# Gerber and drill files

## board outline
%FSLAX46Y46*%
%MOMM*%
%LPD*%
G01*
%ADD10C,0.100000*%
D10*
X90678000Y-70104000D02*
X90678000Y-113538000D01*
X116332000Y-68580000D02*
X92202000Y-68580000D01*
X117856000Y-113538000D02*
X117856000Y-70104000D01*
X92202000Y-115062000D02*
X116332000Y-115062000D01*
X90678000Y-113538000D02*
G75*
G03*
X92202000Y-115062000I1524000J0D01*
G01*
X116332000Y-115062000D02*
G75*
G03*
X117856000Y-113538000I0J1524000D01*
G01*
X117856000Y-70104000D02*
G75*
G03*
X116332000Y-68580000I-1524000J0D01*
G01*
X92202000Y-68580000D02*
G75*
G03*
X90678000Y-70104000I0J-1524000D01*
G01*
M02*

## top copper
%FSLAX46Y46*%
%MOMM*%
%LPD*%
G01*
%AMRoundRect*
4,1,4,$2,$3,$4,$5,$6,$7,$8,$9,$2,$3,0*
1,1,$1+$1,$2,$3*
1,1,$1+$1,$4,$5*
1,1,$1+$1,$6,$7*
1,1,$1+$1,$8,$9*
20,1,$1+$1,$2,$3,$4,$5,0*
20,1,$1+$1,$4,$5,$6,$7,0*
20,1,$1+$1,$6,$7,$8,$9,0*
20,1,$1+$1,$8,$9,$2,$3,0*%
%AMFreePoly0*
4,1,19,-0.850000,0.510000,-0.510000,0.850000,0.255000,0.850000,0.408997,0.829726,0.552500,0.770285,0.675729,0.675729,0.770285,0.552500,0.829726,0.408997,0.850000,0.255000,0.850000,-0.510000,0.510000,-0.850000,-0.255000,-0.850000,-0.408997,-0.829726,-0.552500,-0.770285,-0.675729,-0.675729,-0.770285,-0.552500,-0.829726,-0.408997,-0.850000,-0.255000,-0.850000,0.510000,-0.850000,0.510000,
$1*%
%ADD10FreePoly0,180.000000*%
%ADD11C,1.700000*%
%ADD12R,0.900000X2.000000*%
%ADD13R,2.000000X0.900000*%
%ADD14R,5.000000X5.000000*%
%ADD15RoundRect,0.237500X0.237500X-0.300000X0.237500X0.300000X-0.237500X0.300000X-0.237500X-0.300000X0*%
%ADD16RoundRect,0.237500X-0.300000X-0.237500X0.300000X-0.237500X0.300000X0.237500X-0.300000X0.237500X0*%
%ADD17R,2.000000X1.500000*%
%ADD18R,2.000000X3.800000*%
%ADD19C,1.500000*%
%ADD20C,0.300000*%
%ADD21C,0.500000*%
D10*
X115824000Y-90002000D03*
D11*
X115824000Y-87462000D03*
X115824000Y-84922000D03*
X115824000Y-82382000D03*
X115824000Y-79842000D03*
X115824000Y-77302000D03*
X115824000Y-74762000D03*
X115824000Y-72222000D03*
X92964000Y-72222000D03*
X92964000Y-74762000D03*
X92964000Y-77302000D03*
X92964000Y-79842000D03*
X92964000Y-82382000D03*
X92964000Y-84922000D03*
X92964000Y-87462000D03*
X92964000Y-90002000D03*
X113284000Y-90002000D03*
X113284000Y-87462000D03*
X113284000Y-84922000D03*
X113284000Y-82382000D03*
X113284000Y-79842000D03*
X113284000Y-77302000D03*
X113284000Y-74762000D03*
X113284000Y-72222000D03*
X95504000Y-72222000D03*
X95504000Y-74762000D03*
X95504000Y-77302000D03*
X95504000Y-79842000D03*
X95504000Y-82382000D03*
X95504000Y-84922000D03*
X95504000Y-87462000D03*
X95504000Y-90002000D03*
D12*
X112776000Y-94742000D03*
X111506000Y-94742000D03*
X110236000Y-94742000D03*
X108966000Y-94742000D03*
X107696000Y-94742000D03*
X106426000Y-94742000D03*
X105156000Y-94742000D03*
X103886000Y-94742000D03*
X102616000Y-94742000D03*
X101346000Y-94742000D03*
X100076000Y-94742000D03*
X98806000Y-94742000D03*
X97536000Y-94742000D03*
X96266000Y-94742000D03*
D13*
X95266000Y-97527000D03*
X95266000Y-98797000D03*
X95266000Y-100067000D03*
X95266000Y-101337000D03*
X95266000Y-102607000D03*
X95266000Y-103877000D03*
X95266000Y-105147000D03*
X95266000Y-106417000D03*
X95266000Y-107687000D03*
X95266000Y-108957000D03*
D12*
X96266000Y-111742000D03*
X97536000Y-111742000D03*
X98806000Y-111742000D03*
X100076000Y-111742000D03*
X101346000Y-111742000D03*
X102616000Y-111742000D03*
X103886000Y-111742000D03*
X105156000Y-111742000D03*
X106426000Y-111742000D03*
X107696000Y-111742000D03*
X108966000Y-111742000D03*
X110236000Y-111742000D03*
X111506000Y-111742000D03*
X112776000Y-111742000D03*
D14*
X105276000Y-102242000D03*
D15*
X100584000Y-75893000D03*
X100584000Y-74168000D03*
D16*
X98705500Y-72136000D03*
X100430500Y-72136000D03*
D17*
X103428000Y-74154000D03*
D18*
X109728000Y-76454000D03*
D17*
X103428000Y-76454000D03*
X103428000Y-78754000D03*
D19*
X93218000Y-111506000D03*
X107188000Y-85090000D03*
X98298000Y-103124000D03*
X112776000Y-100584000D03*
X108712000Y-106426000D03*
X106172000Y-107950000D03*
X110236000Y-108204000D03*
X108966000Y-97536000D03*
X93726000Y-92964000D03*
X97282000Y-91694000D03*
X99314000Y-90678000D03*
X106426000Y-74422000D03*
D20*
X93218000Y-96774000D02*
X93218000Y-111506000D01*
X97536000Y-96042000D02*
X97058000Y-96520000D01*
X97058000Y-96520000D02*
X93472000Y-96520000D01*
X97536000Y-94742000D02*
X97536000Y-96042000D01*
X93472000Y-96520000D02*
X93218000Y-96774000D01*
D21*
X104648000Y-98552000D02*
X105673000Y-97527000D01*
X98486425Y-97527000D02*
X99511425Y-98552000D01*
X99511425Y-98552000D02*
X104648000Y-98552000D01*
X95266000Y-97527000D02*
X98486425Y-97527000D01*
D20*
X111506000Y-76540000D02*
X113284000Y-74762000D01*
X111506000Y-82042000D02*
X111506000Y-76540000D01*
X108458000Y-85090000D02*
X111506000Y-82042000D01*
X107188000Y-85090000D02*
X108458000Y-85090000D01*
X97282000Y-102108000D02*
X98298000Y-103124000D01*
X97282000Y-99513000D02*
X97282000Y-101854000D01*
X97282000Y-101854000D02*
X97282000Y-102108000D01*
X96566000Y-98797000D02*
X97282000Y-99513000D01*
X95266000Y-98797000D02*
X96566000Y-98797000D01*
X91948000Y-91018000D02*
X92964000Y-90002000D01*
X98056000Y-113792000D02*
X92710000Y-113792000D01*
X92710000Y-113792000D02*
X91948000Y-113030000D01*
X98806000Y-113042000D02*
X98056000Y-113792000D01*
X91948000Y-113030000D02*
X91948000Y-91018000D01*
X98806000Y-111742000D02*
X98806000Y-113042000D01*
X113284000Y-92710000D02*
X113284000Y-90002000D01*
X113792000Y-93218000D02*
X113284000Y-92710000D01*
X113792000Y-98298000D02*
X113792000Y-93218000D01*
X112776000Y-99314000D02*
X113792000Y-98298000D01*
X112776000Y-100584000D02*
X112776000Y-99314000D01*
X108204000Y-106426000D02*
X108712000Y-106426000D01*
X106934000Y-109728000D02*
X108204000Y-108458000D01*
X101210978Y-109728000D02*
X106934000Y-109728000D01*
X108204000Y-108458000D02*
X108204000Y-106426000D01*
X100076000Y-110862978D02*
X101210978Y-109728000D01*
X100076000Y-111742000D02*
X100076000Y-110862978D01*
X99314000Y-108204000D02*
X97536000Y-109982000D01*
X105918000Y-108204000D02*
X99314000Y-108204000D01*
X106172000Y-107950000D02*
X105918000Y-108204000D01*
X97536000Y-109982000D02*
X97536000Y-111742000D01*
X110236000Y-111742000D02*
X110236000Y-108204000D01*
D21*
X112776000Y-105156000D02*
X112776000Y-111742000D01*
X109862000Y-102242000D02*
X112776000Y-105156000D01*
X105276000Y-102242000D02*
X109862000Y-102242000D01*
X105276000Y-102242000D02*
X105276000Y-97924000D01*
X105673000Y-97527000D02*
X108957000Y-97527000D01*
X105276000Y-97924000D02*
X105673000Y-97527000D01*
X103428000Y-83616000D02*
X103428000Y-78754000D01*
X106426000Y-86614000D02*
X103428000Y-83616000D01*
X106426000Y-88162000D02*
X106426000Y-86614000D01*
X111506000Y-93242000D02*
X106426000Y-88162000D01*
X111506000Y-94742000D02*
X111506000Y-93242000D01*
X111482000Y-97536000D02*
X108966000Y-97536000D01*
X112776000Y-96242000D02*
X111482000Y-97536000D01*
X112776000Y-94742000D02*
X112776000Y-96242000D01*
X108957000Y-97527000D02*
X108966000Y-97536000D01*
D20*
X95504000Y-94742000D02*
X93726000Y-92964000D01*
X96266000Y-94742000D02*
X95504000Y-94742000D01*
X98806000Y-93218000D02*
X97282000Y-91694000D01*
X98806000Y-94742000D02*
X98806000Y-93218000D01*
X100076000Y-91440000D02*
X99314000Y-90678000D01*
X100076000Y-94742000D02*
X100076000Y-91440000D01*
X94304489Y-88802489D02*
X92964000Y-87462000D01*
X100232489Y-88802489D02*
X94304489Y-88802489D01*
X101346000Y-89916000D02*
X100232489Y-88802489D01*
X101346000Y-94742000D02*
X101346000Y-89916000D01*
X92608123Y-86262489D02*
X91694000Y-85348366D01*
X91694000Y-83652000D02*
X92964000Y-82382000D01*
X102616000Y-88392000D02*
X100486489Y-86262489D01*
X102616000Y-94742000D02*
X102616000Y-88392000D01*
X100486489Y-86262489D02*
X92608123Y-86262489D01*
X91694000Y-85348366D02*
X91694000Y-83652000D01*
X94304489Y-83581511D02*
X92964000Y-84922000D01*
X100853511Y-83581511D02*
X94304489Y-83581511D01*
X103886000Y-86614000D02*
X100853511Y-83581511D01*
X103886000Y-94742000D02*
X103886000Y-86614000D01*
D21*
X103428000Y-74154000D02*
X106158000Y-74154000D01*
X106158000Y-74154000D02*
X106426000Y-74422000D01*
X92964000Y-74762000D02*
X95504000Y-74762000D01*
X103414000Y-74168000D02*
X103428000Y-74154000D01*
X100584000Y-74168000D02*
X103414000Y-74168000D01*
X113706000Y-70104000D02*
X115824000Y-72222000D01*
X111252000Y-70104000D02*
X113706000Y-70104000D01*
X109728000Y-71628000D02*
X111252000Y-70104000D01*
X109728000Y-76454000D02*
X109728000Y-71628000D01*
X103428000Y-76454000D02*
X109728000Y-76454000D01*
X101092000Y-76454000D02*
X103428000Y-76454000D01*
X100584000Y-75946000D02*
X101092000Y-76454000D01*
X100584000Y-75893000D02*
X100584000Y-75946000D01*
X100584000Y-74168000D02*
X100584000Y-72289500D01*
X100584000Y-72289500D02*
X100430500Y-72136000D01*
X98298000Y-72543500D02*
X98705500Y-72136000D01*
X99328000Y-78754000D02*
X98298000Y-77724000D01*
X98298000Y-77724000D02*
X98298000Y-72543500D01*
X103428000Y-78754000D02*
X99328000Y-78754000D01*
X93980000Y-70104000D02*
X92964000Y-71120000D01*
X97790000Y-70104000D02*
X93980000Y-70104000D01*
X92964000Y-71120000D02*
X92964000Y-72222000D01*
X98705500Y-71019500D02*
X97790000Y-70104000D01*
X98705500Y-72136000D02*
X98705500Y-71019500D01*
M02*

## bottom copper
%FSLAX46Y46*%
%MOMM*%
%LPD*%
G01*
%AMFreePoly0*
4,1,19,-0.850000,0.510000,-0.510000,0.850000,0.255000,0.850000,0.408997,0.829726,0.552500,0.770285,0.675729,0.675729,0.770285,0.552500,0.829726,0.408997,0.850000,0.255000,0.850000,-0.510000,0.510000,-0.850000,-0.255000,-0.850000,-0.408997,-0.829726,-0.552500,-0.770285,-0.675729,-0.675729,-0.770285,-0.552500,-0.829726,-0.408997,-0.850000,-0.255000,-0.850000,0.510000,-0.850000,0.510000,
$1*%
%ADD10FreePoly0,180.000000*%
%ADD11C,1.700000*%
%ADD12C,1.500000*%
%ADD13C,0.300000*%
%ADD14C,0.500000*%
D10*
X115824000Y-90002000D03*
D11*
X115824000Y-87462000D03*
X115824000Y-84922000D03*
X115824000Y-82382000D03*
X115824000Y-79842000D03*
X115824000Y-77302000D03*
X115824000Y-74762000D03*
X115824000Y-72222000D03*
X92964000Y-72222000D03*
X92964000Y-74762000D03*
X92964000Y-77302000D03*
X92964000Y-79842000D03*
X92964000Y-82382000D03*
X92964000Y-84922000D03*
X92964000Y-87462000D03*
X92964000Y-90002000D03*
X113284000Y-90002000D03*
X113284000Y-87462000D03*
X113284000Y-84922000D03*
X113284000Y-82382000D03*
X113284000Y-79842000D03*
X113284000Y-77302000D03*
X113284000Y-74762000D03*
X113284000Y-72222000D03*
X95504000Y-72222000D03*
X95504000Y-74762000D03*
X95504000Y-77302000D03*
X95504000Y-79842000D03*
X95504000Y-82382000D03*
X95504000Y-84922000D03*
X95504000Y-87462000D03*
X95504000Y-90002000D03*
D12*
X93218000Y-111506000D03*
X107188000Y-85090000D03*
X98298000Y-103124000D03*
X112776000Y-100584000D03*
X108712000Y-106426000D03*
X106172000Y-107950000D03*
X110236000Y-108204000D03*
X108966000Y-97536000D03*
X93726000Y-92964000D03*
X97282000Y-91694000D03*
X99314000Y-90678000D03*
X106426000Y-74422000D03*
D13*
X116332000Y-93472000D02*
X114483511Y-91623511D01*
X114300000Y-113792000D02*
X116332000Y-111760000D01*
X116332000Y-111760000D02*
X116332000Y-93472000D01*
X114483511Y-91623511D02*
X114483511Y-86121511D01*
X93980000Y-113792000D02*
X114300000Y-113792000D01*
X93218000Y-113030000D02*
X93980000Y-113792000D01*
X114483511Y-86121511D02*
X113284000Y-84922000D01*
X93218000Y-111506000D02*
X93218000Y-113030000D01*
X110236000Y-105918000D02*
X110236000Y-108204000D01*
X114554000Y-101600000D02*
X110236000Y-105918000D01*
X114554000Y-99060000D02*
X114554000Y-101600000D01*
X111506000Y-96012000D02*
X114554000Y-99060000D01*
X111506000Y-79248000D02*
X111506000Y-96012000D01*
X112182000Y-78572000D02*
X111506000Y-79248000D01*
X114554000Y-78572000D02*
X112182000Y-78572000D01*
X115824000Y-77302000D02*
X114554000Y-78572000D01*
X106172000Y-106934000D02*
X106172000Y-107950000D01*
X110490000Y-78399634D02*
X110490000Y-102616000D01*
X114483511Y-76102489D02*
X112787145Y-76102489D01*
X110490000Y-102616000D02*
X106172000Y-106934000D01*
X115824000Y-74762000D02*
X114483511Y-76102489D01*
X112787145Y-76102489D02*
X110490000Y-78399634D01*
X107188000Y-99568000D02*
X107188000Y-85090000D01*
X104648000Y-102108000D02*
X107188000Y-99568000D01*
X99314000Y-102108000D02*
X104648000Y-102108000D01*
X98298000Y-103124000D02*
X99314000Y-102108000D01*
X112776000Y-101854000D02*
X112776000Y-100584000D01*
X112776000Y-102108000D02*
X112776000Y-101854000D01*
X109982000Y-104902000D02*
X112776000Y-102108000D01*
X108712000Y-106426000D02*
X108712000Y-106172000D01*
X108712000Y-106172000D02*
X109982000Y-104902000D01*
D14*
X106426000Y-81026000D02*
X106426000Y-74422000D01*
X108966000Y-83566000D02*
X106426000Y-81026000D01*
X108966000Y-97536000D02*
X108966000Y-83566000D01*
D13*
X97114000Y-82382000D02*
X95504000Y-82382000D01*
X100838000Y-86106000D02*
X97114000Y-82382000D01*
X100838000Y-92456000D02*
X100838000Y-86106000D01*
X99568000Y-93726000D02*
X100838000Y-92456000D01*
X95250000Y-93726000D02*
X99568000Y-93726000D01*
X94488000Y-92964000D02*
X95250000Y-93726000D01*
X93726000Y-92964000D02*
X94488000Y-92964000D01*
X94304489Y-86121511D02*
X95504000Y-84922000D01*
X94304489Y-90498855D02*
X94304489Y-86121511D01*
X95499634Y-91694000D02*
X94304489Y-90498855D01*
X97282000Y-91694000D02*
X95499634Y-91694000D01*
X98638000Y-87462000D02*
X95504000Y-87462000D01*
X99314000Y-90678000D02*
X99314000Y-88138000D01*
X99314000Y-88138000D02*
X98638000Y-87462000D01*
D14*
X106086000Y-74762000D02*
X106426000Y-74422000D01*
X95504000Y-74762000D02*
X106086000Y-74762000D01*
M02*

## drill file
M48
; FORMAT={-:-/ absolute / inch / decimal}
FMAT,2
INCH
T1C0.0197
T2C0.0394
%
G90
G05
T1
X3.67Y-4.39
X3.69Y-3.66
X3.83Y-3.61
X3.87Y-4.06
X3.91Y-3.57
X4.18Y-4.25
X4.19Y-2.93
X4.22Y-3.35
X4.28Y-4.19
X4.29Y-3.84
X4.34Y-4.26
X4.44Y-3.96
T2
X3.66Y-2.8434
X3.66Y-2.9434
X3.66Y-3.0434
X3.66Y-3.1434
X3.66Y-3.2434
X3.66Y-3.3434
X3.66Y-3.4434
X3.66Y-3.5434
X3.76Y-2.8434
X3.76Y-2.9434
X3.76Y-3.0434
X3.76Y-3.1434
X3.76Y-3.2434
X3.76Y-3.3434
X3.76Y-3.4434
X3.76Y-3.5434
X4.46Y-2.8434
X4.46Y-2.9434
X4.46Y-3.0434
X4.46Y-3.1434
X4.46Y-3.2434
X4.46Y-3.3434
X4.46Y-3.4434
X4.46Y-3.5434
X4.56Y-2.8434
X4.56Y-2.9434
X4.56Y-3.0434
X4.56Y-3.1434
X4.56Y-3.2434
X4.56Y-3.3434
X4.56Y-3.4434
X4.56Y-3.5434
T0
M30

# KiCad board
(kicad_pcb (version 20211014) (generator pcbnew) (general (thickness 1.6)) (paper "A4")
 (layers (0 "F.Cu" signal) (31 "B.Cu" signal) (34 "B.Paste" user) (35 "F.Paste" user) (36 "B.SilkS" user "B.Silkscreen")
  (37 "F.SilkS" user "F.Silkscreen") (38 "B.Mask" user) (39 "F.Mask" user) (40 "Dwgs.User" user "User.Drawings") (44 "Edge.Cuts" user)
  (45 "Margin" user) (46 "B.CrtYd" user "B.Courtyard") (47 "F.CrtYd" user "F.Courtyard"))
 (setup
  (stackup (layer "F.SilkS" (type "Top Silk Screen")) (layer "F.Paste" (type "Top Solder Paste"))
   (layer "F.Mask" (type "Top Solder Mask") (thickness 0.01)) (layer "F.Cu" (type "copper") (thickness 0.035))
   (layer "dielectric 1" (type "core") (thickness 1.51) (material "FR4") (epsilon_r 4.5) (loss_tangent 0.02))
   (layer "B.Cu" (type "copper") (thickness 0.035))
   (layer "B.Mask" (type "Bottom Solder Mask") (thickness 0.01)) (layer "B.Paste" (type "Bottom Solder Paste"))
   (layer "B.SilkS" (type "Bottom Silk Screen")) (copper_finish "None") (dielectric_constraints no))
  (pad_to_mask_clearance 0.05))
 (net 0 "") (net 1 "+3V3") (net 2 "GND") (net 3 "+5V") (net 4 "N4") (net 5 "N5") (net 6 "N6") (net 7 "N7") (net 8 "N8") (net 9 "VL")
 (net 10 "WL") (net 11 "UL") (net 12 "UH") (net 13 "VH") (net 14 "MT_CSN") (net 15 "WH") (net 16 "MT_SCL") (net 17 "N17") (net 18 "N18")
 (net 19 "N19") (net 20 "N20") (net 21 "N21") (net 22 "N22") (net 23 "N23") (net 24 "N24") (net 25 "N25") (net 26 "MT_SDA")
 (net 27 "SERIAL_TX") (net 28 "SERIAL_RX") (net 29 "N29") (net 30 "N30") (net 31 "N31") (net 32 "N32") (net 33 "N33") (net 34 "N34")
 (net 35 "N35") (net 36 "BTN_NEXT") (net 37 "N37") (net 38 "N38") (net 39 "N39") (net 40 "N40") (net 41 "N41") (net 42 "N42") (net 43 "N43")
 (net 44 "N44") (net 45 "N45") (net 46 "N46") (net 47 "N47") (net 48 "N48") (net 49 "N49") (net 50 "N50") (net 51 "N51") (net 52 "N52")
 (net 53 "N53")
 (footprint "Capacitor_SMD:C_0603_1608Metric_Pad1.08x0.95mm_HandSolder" (layer "F.Cu") (at 100.584 75.0305 90)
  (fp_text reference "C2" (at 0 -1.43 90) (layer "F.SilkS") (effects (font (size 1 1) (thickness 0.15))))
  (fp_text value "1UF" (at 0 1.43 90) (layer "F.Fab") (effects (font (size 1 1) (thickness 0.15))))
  (pad "1" smd roundrect (at -0.8625 0 90) (size 1.075 0.95) (layers "F.Cu" "F.Paste" "F.Mask") (roundrect_rratio 0.25) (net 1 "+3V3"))
  (pad "2" smd roundrect (at 0.8625 0 90) (size 1.075 0.95) (layers "F.Cu" "F.Paste" "F.Mask") (roundrect_rratio 0.25) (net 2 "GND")))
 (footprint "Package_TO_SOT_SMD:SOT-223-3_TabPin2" (layer "F.Cu") (at 106.578 76.454)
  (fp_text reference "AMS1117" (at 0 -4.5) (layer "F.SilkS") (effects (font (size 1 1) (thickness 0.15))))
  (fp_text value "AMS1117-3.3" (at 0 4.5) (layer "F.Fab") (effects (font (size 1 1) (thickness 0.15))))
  (pad "1" smd rect (at -3.15 -2.3) (size 2 1.5) (layers "F.Cu" "F.Paste" "F.Mask") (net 2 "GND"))
  (pad "2" smd rect (at -3.15 0) (size 2 1.5) (layers "F.Cu" "F.Paste" "F.Mask") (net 1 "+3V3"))
  (pad "2" smd rect (at 3.15 0) (size 2 3.8) (layers "F.Cu" "F.Paste" "F.Mask") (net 1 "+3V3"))
  (pad "3" smd rect (at -3.15 2.3) (size 2 1.5) (layers "F.Cu" "F.Paste" "F.Mask") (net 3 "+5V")))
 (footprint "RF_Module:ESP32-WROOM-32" (layer "F.Cu") (at 104.521 103.242 -90)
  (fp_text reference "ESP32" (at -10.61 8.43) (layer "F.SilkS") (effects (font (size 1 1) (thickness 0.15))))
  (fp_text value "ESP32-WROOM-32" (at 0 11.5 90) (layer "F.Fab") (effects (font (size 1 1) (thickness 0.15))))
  (pad "1" smd rect (at -8.5 -8.255 270) (size 2 0.9) (layers "F.Cu" "F.Paste" "F.Mask") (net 2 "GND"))
  (pad "2" smd rect (at -8.5 -6.985 270) (size 2 0.9) (layers "F.Cu" "F.Paste" "F.Mask") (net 3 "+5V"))
  (pad "3" smd rect (at -8.5 -5.715 270) (size 2 0.9) (layers "F.Cu" "F.Paste" "F.Mask") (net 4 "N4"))
  (pad "4" smd rect (at -8.5 -4.445 270) (size 2 0.9) (layers "F.Cu" "F.Paste" "F.Mask") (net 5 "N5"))
  (pad "5" smd rect (at -8.5 -3.175 270) (size 2 0.9) (layers "F.Cu" "F.Paste" "F.Mask") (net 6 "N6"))
  (pad "6" smd rect (at -8.5 -1.905 270) (size 2 0.9) (layers "F.Cu" "F.Paste" "F.Mask") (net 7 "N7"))
  (pad "7" smd rect (at -8.5 -0.635 270) (size 2 0.9) (layers "F.Cu" "F.Paste" "F.Mask") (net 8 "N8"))
  (pad "8" smd rect (at -8.5 0.635 270) (size 2 0.9) (layers "F.Cu" "F.Paste" "F.Mask") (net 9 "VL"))
  (pad "9" smd rect (at -8.5 1.905 270) (size 2 0.9) (layers "F.Cu" "F.Paste" "F.Mask") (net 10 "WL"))
  (pad "10" smd rect (at -8.5 3.175 270) (size 2 0.9) (layers "F.Cu" "F.Paste" "F.Mask") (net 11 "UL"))
  (pad "11" smd rect (at -8.5 4.445 270) (size 2 0.9) (layers "F.Cu" "F.Paste" "F.Mask") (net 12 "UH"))
  (pad "12" smd rect (at -8.5 5.715 270) (size 2 0.9) (layers "F.Cu" "F.Paste" "F.Mask") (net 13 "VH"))
  (pad "13" smd rect (at -8.5 6.985 270) (size 2 0.9) (layers "F.Cu" "F.Paste" "F.Mask") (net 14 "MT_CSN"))
  (pad "14" smd rect (at -8.5 8.255 270) (size 2 0.9) (layers "F.Cu" "F.Paste" "F.Mask") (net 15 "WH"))
  (pad "15" smd rect (at -5.715 9.255) (size 2 0.9) (layers "F.Cu" "F.Paste" "F.Mask") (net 2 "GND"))
  (pad "16" smd rect (at -4.445 9.255) (size 2 0.9) (layers "F.Cu" "F.Paste" "F.Mask") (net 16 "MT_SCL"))
  (pad "17" smd rect (at -3.175 9.255) (size 2 0.9) (layers "F.Cu" "F.Paste" "F.Mask") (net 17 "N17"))
  (pad "18" smd rect (at -1.905 9.255) (size 2 0.9) (layers "F.Cu" "F.Paste" "F.Mask") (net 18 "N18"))
  (pad "19" smd rect (at -0.635 9.255) (size 2 0.9) (layers "F.Cu" "F.Paste" "F.Mask") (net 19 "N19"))
  (pad "20" smd rect (at 0.635 9.255) (size 2 0.9) (layers "F.Cu" "F.Paste" "F.Mask") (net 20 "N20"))
  (pad "21" smd rect (at 1.905 9.255) (size 2 0.9) (layers "F.Cu" "F.Paste" "F.Mask") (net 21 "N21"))
  (pad "22" smd rect (at 3.175 9.255) (size 2 0.9) (layers "F.Cu" "F.Paste" "F.Mask") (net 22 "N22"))
  (pad "23" smd rect (at 4.445 9.255) (size 2 0.9) (layers "F.Cu" "F.Paste" "F.Mask") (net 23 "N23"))
  (pad "24" smd rect (at 5.715 9.255) (size 2 0.9) (layers "F.Cu" "F.Paste" "F.Mask") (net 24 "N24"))
  (pad "25" smd rect (at 8.5 8.255 270) (size 2 0.9) (layers "F.Cu" "F.Paste" "F.Mask") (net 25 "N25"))
  (pad "26" smd rect (at 8.5 6.985 270) (size 2 0.9) (layers "F.Cu" "F.Paste" "F.Mask") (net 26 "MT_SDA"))
  (pad "27" smd rect (at 8.5 5.715 270) (size 2 0.9) (layers "F.Cu" "F.Paste" "F.Mask") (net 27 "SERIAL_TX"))
  (pad "28" smd rect (at 8.5 4.445 270) (size 2 0.9) (layers "F.Cu" "F.Paste" "F.Mask") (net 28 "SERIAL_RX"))
  (pad "29" smd rect (at 8.5 3.175 270) (size 2 0.9) (layers "F.Cu" "F.Paste" "F.Mask") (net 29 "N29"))
  (pad "30" smd rect (at 8.5 1.905 270) (size 2 0.9) (layers "F.Cu" "F.Paste" "F.Mask") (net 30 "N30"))
  (pad "31" smd rect (at 8.5 0.635 270) (size 2 0.9) (layers "F.Cu" "F.Paste" "F.Mask") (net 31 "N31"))
  (pad "32" smd rect (at 8.5 -0.635 270) (size 2 0.9) (layers "F.Cu" "F.Paste" "F.Mask") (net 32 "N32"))
  (pad "33" smd rect (at 8.5 -1.905 270) (size 2 0.9) (layers "F.Cu" "F.Paste" "F.Mask") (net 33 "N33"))
  (pad "34" smd rect (at 8.5 -3.175 270) (size 2 0.9) (layers "F.Cu" "F.Paste" "F.Mask") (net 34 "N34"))
  (pad "35" smd rect (at 8.5 -4.445 270) (size 2 0.9) (layers "F.Cu" "F.Paste" "F.Mask") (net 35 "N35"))
  (pad "36" smd rect (at 8.5 -5.715 270) (size 2 0.9) (layers "F.Cu" "F.Paste" "F.Mask") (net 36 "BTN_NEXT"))
  (pad "37" smd rect (at 8.5 -6.985 270) (size 2 0.9) (layers "F.Cu" "F.Paste" "F.Mask") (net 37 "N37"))
  (pad "38" smd rect (at 8.5 -8.255 270) (size 2 0.9) (layers "F.Cu" "F.Paste" "F.Mask") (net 2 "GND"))
  (pad "39" smd rect (at -1 -0.755 270) (size 5 5) (layers "F.Cu" "F.Paste" "F.Mask") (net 2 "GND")))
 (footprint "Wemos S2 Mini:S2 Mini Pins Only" (layer "F.Cu") (at 104.394 79.502 180)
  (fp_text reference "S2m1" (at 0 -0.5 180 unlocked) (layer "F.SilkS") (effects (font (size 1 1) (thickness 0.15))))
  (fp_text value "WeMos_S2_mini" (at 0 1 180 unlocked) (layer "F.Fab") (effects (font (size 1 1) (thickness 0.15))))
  (pad "1" thru_hole roundrect (at -11.43 -10.5 180) (size 1.7 1.7) (drill 1) (layers *.Cu *.Mask) (roundrect_rratio 0.35)
   (chamfer_ratio 0.2) (chamfer top_left bottom_right) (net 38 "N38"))
  (pad "2" thru_hole circle (at -11.43 -7.96 180) (size 1.7 1.7) (drill 1) (layers *.Cu *.Mask) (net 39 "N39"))
  (pad "3" thru_hole circle (at -11.43 -5.42 180) (size 1.7 1.7) (drill 1) (layers *.Cu *.Mask) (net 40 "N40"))
  (pad "4" thru_hole circle (at -11.43 -2.88 180) (size 1.7 1.7) (drill 1) (layers *.Cu *.Mask) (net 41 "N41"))
  (pad "5" thru_hole circle (at -11.43 -0.34 180) (size 1.7 1.7) (drill 1) (layers *.Cu *.Mask) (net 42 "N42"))
  (pad "6" thru_hole circle (at -11.43 2.2 180) (size 1.7 1.7) (drill 1) (layers *.Cu *.Mask) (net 36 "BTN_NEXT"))
  (pad "7" thru_hole circle (at -11.43 4.74 180) (size 1.7 1.7) (drill 1) (layers *.Cu *.Mask) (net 26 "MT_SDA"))
  (pad "8" thru_hole circle (at -11.43 7.28 180) (size 1.7 1.7) (drill 1) (layers *.Cu *.Mask) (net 1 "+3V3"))
  (pad "9" thru_hole circle (at 11.43 7.28 180) (size 1.7 1.7) (drill 1) (layers *.Cu *.Mask) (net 3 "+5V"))
  (pad "10" thru_hole circle (at 11.43 4.74 180) (size 1.7 1.7) (drill 1) (layers *.Cu *.Mask) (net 2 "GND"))
  (pad "11" thru_hole circle (at 11.43 2.2 180) (size 1.7 1.7) (drill 1) (layers *.Cu *.Mask) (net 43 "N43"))
  (pad "12" thru_hole circle (at 11.43 -0.34 180) (size 1.7 1.7) (drill 1) (layers *.Cu *.Mask) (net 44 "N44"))
  (pad "13" thru_hole circle (at 11.43 -2.88 180) (size 1.7 1.7) (drill 1) (layers *.Cu *.Mask) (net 10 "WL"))
  (pad "14" thru_hole circle (at 11.43 -5.42 180) (size 1.7 1.7) (drill 1) (layers *.Cu *.Mask) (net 9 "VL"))
  (pad "15" thru_hole circle (at 11.43 -7.96 180) (size 1.7 1.7) (drill 1) (layers *.Cu *.Mask) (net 11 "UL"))
  (pad "16" thru_hole circle (at 11.43 -10.5 180) (size 1.7 1.7) (drill 1) (layers *.Cu *.Mask) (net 27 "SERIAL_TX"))
  (pad "17" thru_hole circle (at -8.89 -10.5 180) (size 1.7 1.7) (drill 1) (layers *.Cu *.Mask) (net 28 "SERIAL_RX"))
  (pad "18" thru_hole circle (at -8.89 -7.96 180) (size 1.7 1.7) (drill 1) (layers *.Cu *.Mask) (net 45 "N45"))
  (pad "19" thru_hole circle (at -8.89 -5.42 180) (size 1.7 1.7) (drill 1) (layers *.Cu *.Mask) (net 14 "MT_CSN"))
  (pad "20" thru_hole circle (at -8.89 -2.88 180) (size 1.7 1.7) (drill 1) (layers *.Cu *.Mask) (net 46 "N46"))
  (pad "21" thru_hole circle (at -8.89 -0.34 180) (size 1.7 1.7) (drill 1) (layers *.Cu *.Mask) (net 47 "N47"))
  (pad "22" thru_hole circle (at -8.89 2.2 180) (size 1.7 1.7) (drill 1) (layers *.Cu *.Mask) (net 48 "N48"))
  (pad "23" thru_hole circle (at -8.89 4.74 180) (size 1.7 1.7) (drill 1) (layers *.Cu *.Mask) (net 16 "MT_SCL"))
  (pad "24" thru_hole circle (at -8.89 7.28 180) (size 1.7 1.7) (drill 1) (layers *.Cu *.Mask) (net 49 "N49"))
  (pad "25" thru_hole circle (at 8.89 7.28 180) (size 1.7 1.7) (drill 1) (layers *.Cu *.Mask) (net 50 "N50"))
  (pad "26" thru_hole circle (at 8.89 4.74 180) (size 1.7 1.7) (drill 1) (layers *.Cu *.Mask) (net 2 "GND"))
  (pad "27" thru_hole circle (at 8.89 2.2 180) (size 1.7 1.7) (drill 1) (layers *.Cu *.Mask) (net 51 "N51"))
  (pad "28" thru_hole circle (at 8.89 -0.34 180) (size 1.7 1.7) (drill 1) (layers *.Cu *.Mask) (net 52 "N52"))
  (pad "29" thru_hole circle (at 8.89 -2.88 180) (size 1.7 1.7) (drill 1) (layers *.Cu *.Mask) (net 15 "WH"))
  (pad "30" thru_hole circle (at 8.89 -5.42 180) (size 1.7 1.7) (drill 1) (layers *.Cu *.Mask) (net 13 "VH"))
  (pad "31" thru_hole circle (at 8.89 -7.96 180) (size 1.7 1.7) (drill 1) (layers *.Cu *.Mask) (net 12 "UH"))
  (pad "32" thru_hole circle (at 8.89 -10.5 180) (size 1.7 1.7) (drill 1) (layers *.Cu *.Mask) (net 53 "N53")))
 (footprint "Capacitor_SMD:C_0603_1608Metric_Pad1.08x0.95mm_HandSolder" (layer "F.Cu") (at 99.568 72.136)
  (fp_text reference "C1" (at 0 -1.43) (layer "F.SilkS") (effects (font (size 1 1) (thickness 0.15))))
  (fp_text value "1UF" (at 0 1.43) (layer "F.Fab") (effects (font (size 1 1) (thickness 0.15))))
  (pad "1" smd roundrect (at -0.8625 0) (size 1.075 0.95) (layers "F.Cu" "F.Paste" "F.Mask") (roundrect_rratio 0.25) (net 3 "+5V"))
  (pad "2" smd roundrect (at 0.8625 0) (size 1.075 0.95) (layers "F.Cu" "F.Paste" "F.Mask") (roundrect_rratio 0.25) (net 2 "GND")))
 (gr_arc (start 117.856 113.538) (mid 117.409631 114.615631) (end 116.332 115.062) (layer "Edge.Cuts") (width 0.1))
 (gr_arc (start 90.678 70.104) (mid 91.124369 69.026369) (end 92.202 68.58) (layer "Edge.Cuts") (width 0.1))
 (gr_line (start 90.678 70.104) (end 90.678 113.538) (layer "Edge.Cuts") (width 0.1))
 (gr_arc (start 116.332 68.58) (mid 117.409631 69.026369) (end 117.856 70.104) (layer "Edge.Cuts") (width 0.1))
 (gr_line (start 92.202 115.062) (end 116.332 115.062) (layer "Edge.Cuts") (width 0.1))
 (gr_line (start 117.856 113.538) (end 117.856 70.104) (layer "Edge.Cuts") (width 0.1))
 (gr_line (start 116.332 68.58) (end 92.202 68.58) (layer "Edge.Cuts") (width 0.1))
 (gr_arc (start 92.202 115.062) (mid 91.124369 114.615631) (end 90.678 113.538) (layer "Edge.Cuts") (width 0.1))
 (segment (start 106.158 74.154) (end 106.426 74.422) (width 0.5) (layer "F.Cu") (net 2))
 (segment (start 99.511425 98.552) (end 104.648 98.552) (width 0.5) (layer "F.Cu") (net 2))
 (segment (start 98.486425 97.527) (end 99.511425 98.552) (width 0.5) (layer "F.Cu") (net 2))
 (segment (start 103.414 74.168) (end 103.428 74.154) (width 0.5) (layer "F.Cu") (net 2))
 (segment (start 112.776 105.156) (end 112.776 111.742) (width 0.5) (layer "F.Cu") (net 2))
 (segment (start 105.276 97.924) (end 105.673 97.527) (width 0.5) (layer "F.Cu") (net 2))
 (segment (start 100.584 74.168) (end 100.584 72.2895) (width 0.5) (layer "F.Cu") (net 2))
 (segment (start 104.648 98.552) (end 105.673 97.527) (width 0.5) (layer "F.Cu") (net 2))
 (segment (start 105.673 97.527) (end 108.957 97.527) (width 0.5) (layer "F.Cu") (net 2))
 (segment (start 100.584 72.2895) (end 100.4305 72.136) (width 0.5) (layer "F.Cu") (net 2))
 (segment (start 103.428 74.154) (end 106.158 74.154) (width 0.5) (layer "F.Cu") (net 2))
 (segment (start 112.776 96.242) (end 111.482 97.536) (width 0.5) (layer "F.Cu") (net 2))
 (segment (start 109.862 102.242) (end 112.776 105.156) (width 0.5) (layer "F.Cu") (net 2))
 (segment (start 111.482 97.536) (end 108.966 97.536) (width 0.5) (layer "F.Cu") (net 2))
 (segment (start 92.964 74.762) (end 95.504 74.762) (width 0.5) (layer "F.Cu") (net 2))
 (segment (start 112.776 94.742) (end 112.776 96.242) (width 0.5) (layer "F.Cu") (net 2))
 (segment (start 108.957 97.527) (end 108.966 97.536) (width 0.5) (layer "F.Cu") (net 2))
 (segment (start 100.584 74.168) (end 103.414 74.168) (width 0.5) (layer "F.Cu") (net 2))
 (segment (start 95.266 97.527) (end 98.486425 97.527) (width 0.5) (layer "F.Cu") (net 2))
 (segment (start 105.276 102.242) (end 105.276 97.924) (width 0.5) (layer "F.Cu") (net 2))
 (segment (start 105.276 102.242) (end 109.862 102.242) (width 0.5) (layer "F.Cu") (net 2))
 (via (at 106.426 74.422) (size 1.5) (drill 0.5) (layers "F.Cu" "B.Cu") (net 2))
 (via (at 108.966 97.536) (size 1.5) (drill 0.5) (layers "F.Cu" "B.Cu") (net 2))
 (segment (start 106.086 74.762) (end 106.426 74.422) (width 0.5) (layer "B.Cu") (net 2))
 (segment (start 108.966 97.536) (end 108.966 83.566) (width 0.5) (layer "B.Cu") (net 2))
 (segment (start 95.504 74.762) (end 106.086 74.762) (width 0.5) (layer "B.Cu") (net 2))
 (segment (start 108.966 83.566) (end 106.426 81.026) (width 0.5) (layer "B.Cu") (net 2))
 (segment (start 106.426 81.026) (end 106.426 74.422) (width 0.5) (layer "B.Cu") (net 2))
 (segment (start 109.728 76.454) (end 109.728 71.628) (width 0.5) (layer "F.Cu") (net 1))
 (segment (start 111.252 70.104) (end 113.706 70.104) (width 0.5) (layer "F.Cu") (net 1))
 (segment (start 109.728 71.628) (end 111.252 70.104) (width 0.5) (layer "F.Cu") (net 1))
 (segment (start 101.092 76.454) (end 103.428 76.454) (width 0.5) (layer "F.Cu") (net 1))
 (segment (start 103.428 76.454) (end 109.728 76.454) (width 0.5) (layer "F.Cu") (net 1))
 (segment (start 100.584 75.893) (end 100.584 75.946) (width 0.5) (layer "F.Cu") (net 1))
 (segment (start 100.584 75.946) (end 101.092 76.454) (width 0.5) (layer "F.Cu") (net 1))
 (segment (start 113.706 70.104) (end 115.824 72.222) (width 0.5) (layer "F.Cu") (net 1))
 (segment (start 98.298 77.724) (end 98.298 72.5435) (width 0.5) (layer "F.Cu") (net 3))
 (segment (start 111.506 93.242) (end 106.426 88.162) (width 0.5) (layer "F.Cu") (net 3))
 (segment (start 93.98 70.104) (end 92.964 71.12) (width 0.5) (layer "F.Cu") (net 3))
 (segment (start 106.426 86.614) (end 103.428 83.616) (width 0.5) (layer "F.Cu") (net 3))
 (segment (start 92.964 71.12) (end 92.964 72.222) (width 0.5) (layer "F.Cu") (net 3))
 (segment (start 111.506 94.742) (end 111.506 93.242) (width 0.5) (layer "F.Cu") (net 3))
 (segment (start 98.298 72.5435) (end 98.7055 72.136) (width 0.5) (layer "F.Cu") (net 3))
 (segment (start 103.428 78.754) (end 99.328 78.754) (width 0.5) (layer "F.Cu") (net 3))
 (segment (start 103.428 83.616) (end 103.428 78.754) (width 0.5) (layer "F.Cu") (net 3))
 (segment (start 106.426 88.162) (end 106.426 86.614) (width 0.5) (layer "F.Cu") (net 3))
 (segment (start 98.7055 71.0195) (end 97.79 70.104) (width 0.5) (layer "F.Cu") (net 3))
 (segment (start 98.7055 72.136) (end 98.7055 71.0195) (width 0.5) (layer "F.Cu") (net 3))
 (segment (start 97.79 70.104) (end 93.98 70.104) (width 0.5) (layer "F.Cu") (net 3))
 (segment (start 99.328 78.754) (end 98.298 77.724) (width 0.5) (layer "F.Cu") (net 3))
 (segment (start 100.853511 83.581511) (end 94.304489 83.581511) (width 0.3) (layer "F.Cu") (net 9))
 (segment (start 94.304489 83.581511) (end 92.964 84.922) (width 0.3) (layer "F.Cu") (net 9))
 (segment (start 103.886 86.614) (end 100.853511 83.581511) (width 0.3) (layer "F.Cu") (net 9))
 (segment (start 103.886 94.742) (end 103.886 86.614) (width 0.3) (layer "F.Cu") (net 9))
 (segment (start 92.608123 86.262489) (end 91.694 85.348366) (width 0.3) (layer "F.Cu") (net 10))
 (segment (start 91.694 85.348366) (end 91.694 83.652) (width 0.3) (layer "F.Cu") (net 10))
 (segment (start 91.694 83.652) (end 92.964 82.382) (width 0.3) (layer "F.Cu") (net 10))
 (segment (start 102.616 94.742) (end 102.616 88.392) (width 0.3) (layer "F.Cu") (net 10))
 (segment (start 100.486489 86.262489) (end 92.608123 86.262489) (width 0.3) (layer "F.Cu") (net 10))
 (segment (start 102.616 88.392) (end 100.486489 86.262489) (width 0.3) (layer "F.Cu") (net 10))
 (segment (start 101.346 94.742) (end 101.346 89.916) (width 0.3) (layer "F.Cu") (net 11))
 (segment (start 100.232489 88.802489) (end 94.304489 88.802489) (width 0.3) (layer "F.Cu") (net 11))
 (segment (start 94.304489 88.802489) (end 92.964 87.462) (width 0.3) (layer "F.Cu") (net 11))
 (segment (start 101.346 89.916) (end 100.232489 88.802489) (width 0.3) (layer "F.Cu") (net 11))
 (segment (start 100.076 91.44) (end 99.314 90.678) (width 0.3) (layer "F.Cu") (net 12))
 (segment (start 100.076 94.742) (end 100.076 91.44) (width 0.3) (layer "F.Cu") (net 12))
 (via (at 99.314 90.678) (size 1.5) (drill 0.5) (layers "F.Cu" "B.Cu") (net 12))
 (segment (start 98.638 87.462) (end 95.504 87.462) (width 0.3) (layer "B.Cu") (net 12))
 (segment (start 99.314 88.138) (end 98.638 87.462) (width 0.3) (layer "B.Cu") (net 12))
 (segment (start 99.314 90.678) (end 99.314 88.138) (width 0.3) (layer "B.Cu") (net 12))
 (segment (start 98.806 94.742) (end 98.806 93.218) (width 0.3) (layer "F.Cu") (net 13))
 (segment (start 98.806 93.218) (end 97.282 91.694) (width 0.3) (layer "F.Cu") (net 13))
 (via (at 97.282 91.694) (size 1.5) (drill 0.5) (layers "F.Cu" "B.Cu") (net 13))
 (segment (start 94.304489 90.498855) (end 94.304489 86.121511) (width 0.3) (layer "B.Cu") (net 13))
 (segment (start 95.499634 91.694) (end 94.304489 90.498855) (width 0.3) (layer "B.Cu") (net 13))
 (segment (start 97.282 91.694) (end 95.499634 91.694) (width 0.3) (layer "B.Cu") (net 13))
 (segment (start 94.304489 86.121511) (end 95.504 84.922) (width 0.3) (layer "B.Cu") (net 13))
 (segment (start 97.058 96.52) (end 93.472 96.52) (width 0.3) (layer "F.Cu") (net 14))
 (segment (start 93.472 96.52) (end 93.218 96.774) (width 0.3) (layer "F.Cu") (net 14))
 (segment (start 97.536 96.042) (end 97.058 96.52) (width 0.3) (layer "F.Cu") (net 14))
 (segment (start 97.536 94.742) (end 97.536 96.042) (width 0.3) (layer "F.Cu") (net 14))
 (segment (start 93.218 96.774) (end 93.218 111.506) (width 0.3) (layer "F.Cu") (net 14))
 (via (at 93.218 111.506) (size 1.5) (drill 0.5) (layers "F.Cu" "B.Cu") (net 14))
 (segment (start 93.218 111.506) (end 93.218 113.03) (width 0.3) (layer "B.Cu") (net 14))
 (segment (start 114.3 113.792) (end 116.332 111.76) (width 0.3) (layer "B.Cu") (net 14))
 (segment (start 116.332 93.472) (end 114.483511 91.623511) (width 0.3) (layer "B.Cu") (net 14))
 (segment (start 93.98 113.792) (end 114.3 113.792) (width 0.3) (layer "B.Cu") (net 14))
 (segment (start 114.483511 86.121511) (end 113.284 84.922) (width 0.3) (layer "B.Cu") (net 14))
 (segment (start 93.218 113.03) (end 93.98 113.792) (width 0.3) (layer "B.Cu") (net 14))
 (segment (start 114.483511 91.623511) (end 114.483511 86.121511) (width 0.3) (layer "B.Cu") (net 14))
 (segment (start 116.332 111.76) (end 116.332 93.472) (width 0.3) (layer "B.Cu") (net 14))
 (segment (start 96.266 94.742) (end 95.504 94.742) (width 0.3) (layer "F.Cu") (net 15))
 (segment (start 95.504 94.742) (end 93.726 92.964) (width 0.3) (layer "F.Cu") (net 15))
 (via (at 93.726 92.964) (size 1.5) (drill 0.5) (layers "F.Cu" "B.Cu") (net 15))
 (segment (start 100.838 86.106) (end 97.114 82.382) (width 0.3) (layer "B.Cu") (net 15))
 (segment (start 94.488 92.964) (end 95.25 93.726) (width 0.3) (layer "B.Cu") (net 15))
 (segment (start 99.568 93.726) (end 100.838 92.456) (width 0.3) (layer "B.Cu") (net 15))
 (segment (start 100.838 92.456) (end 100.838 86.106) (width 0.3) (layer "B.Cu") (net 15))
 (segment (start 93.726 92.964) (end 94.488 92.964) (width 0.3) (layer "B.Cu") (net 15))
 (segment (start 95.25 93.726) (end 99.568 93.726) (width 0.3) (layer "B.Cu") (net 15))
 (segment (start 97.114 82.382) (end 95.504 82.382) (width 0.3) (layer "B.Cu") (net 15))
 (segment (start 97.282 102.108) (end 98.298 103.124) (width 0.3) (layer "F.Cu") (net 16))
 (segment (start 111.506 82.042) (end 111.506 76.54) (width 0.3) (layer "F.Cu") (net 16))
 (segment (start 107.188 85.09) (end 108.458 85.09) (width 0.3) (layer "F.Cu") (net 16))
 (segment (start 97.282 101.854) (end 97.282 102.108) (width 0.3) (layer "F.Cu") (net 16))
 (segment (start 111.506 76.54) (end 113.284 74.762) (width 0.3) (layer "F.Cu") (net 16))
 (segment (start 95.266 98.797) (end 96.566 98.797) (width 0.3) (layer "F.Cu") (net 16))
 (segment (start 97.282 99.513) (end 97.282 101.854) (width 0.3) (layer "F.Cu") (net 16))
 (segment (start 108.458 85.09) (end 111.506 82.042) (width 0.3) (layer "F.Cu") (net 16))
 (segment (start 96.566 98.797) (end 97.282 99.513) (width 0.3) (layer "F.Cu") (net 16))
 (via (at 98.298 103.124) (size 1.5) (drill 0.5) (layers "F.Cu" "B.Cu") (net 16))
 (via (at 107.188 85.09) (size 1.5) (drill 0.5) (layers "F.Cu" "B.Cu") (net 16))
 (segment (start 99.314 102.108) (end 104.648 102.108) (width 0.3) (layer "B.Cu") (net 16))
 (segment (start 107.188 99.568) (end 107.188 85.09) (width 0.3) (layer "B.Cu") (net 16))
 (segment (start 104.648 102.108) (end 107.188 99.568) (width 0.3) (layer "B.Cu") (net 16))
 (segment (start 98.298 103.124) (end 99.314 102.108) (width 0.3) (layer "B.Cu") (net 16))
 (segment (start 105.918 108.204) (end 99.314 108.204) (width 0.3) (layer "F.Cu") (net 26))
 (segment (start 97.536 109.982) (end 97.536 111.742) (width 0.3) (layer "F.Cu") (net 26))
 (segment (start 106.172 107.95) (end 105.918 108.204) (width 0.3) (layer "F.Cu") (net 26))
 (segment (start 99.314 108.204) (end 97.536 109.982) (width 0.3) (layer "F.Cu") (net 26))
 (via (at 106.172 107.95) (size 1.5) (drill 0.5) (layers "F.Cu" "B.Cu") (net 26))
 (segment (start 110.49 102.616) (end 106.172 106.934) (width 0.3) (layer "B.Cu") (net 26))
 (segment (start 115.824 74.762) (end 114.483511 76.102489) (width 0.3) (layer "B.Cu") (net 26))
 (segment (start 112.787145 76.102489) (end 110.49 78.399634) (width 0.3) (layer "B.Cu") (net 26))
 (segment (start 114.483511 76.102489) (end 112.787145 76.102489) (width 0.3) (layer "B.Cu") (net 26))
 (segment (start 110.49 78.399634) (end 110.49 102.616) (width 0.3) (layer "B.Cu") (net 26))
 (segment (start 106.172 106.934) (end 106.172 107.95) (width 0.3) (layer "B.Cu") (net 26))
 (segment (start 98.056 113.792) (end 92.71 113.792) (width 0.3) (layer "F.Cu") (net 27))
 (segment (start 92.71 113.792) (end 91.948 113.03) (width 0.3) (layer "F.Cu") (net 27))
 (segment (start 91.948 91.018) (end 92.964 90.002) (width 0.3) (layer "F.Cu") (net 27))
 (segment (start 98.806 113.042) (end 98.056 113.792) (width 0.3) (layer "F.Cu") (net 27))
 (segment (start 98.806 111.742) (end 98.806 113.042) (width 0.3) (layer "F.Cu") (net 27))
 (segment (start 91.948 113.03) (end 91.948 91.018) (width 0.3) (layer "F.Cu") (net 27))
 (segment (start 108.204 108.458) (end 108.204 106.426) (width 0.3) (layer "F.Cu") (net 28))
 (segment (start 112.776 100.584) (end 112.776 99.314) (width 0.3) (layer "F.Cu") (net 28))
 (segment (start 113.284 92.71) (end 113.284 90.002) (width 0.3) (layer "F.Cu") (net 28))
 (segment (start 113.792 98.298) (end 113.792 93.218) (width 0.3) (layer "F.Cu") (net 28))
 (segment (start 112.776 99.314) (end 113.792 98.298) (width 0.3) (layer "F.Cu") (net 28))
 (segment (start 108.204 106.426) (end 108.712 106.426) (width 0.3) (layer "F.Cu") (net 28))
 (segment (start 100.076 110.862978) (end 101.210978 109.728) (width 0.3) (layer "F.Cu") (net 28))
 (segment (start 100.076 111.742) (end 100.076 110.862978) (width 0.3) (layer "F.Cu") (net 28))
 (segment (start 106.934 109.728) (end 108.204 108.458) (width 0.3) (layer "F.Cu") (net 28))
 (segment (start 101.210978 109.728) (end 106.934 109.728) (width 0.3) (layer "F.Cu") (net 28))
 (segment (start 113.792 93.218) (end 113.284 92.71) (width 0.3) (layer "F.Cu") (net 28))
 (via (at 112.776 100.584) (size 1.5) (drill 0.5) (layers "F.Cu" "B.Cu") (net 28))
 (via (at 108.712 106.426) (size 1.5) (drill 0.5) (layers "F.Cu" "B.Cu") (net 28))
 (segment (start 109.982 104.902) (end 112.776 102.108) (width 0.3) (layer "B.Cu") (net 28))
 (segment (start 112.776 102.108) (end 112.776 101.854) (width 0.3) (layer "B.Cu") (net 28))
 (segment (start 112.776 101.854) (end 112.776 100.584) (width 0.3) (layer "B.Cu") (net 28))
 (segment (start 108.712 106.172) (end 109.982 104.902) (width 0.3) (layer "B.Cu") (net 28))
 (segment (start 108.712 106.426) (end 108.712 106.172) (width 0.3) (layer "B.Cu") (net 28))
 (segment (start 110.236 111.742) (end 110.236 108.204) (width 0.3) (layer "F.Cu") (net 36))
 (via (at 110.236 108.204) (size 1.5) (drill 0.5) (layers "F.Cu" "B.Cu") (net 36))
 (segment (start 111.506 79.248) (end 111.506 96.012) (width 0.3) (layer "B.Cu") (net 36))
 (segment (start 114.554 78.572) (end 112.182 78.572) (width 0.3) (layer "B.Cu") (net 36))
 (segment (start 115.824 77.302) (end 114.554 78.572) (width 0.3) (layer "B.Cu") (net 36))
 (segment (start 111.506 96.012) (end 114.554 99.06) (width 0.3) (layer "B.Cu") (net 36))
 (segment (start 112.182 78.572) (end 111.506 79.248) (width 0.3) (layer "B.Cu") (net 36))
 (segment (start 114.554 99.06) (end 114.554 101.6) (width 0.3) (layer "B.Cu") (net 36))
 (segment (start 110.236 105.918) (end 110.236 108.204) (width 0.3) (layer "B.Cu") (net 36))
 (segment (start 114.554 101.6) (end 110.236 105.918) (width 0.3) (layer "B.Cu") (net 36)))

